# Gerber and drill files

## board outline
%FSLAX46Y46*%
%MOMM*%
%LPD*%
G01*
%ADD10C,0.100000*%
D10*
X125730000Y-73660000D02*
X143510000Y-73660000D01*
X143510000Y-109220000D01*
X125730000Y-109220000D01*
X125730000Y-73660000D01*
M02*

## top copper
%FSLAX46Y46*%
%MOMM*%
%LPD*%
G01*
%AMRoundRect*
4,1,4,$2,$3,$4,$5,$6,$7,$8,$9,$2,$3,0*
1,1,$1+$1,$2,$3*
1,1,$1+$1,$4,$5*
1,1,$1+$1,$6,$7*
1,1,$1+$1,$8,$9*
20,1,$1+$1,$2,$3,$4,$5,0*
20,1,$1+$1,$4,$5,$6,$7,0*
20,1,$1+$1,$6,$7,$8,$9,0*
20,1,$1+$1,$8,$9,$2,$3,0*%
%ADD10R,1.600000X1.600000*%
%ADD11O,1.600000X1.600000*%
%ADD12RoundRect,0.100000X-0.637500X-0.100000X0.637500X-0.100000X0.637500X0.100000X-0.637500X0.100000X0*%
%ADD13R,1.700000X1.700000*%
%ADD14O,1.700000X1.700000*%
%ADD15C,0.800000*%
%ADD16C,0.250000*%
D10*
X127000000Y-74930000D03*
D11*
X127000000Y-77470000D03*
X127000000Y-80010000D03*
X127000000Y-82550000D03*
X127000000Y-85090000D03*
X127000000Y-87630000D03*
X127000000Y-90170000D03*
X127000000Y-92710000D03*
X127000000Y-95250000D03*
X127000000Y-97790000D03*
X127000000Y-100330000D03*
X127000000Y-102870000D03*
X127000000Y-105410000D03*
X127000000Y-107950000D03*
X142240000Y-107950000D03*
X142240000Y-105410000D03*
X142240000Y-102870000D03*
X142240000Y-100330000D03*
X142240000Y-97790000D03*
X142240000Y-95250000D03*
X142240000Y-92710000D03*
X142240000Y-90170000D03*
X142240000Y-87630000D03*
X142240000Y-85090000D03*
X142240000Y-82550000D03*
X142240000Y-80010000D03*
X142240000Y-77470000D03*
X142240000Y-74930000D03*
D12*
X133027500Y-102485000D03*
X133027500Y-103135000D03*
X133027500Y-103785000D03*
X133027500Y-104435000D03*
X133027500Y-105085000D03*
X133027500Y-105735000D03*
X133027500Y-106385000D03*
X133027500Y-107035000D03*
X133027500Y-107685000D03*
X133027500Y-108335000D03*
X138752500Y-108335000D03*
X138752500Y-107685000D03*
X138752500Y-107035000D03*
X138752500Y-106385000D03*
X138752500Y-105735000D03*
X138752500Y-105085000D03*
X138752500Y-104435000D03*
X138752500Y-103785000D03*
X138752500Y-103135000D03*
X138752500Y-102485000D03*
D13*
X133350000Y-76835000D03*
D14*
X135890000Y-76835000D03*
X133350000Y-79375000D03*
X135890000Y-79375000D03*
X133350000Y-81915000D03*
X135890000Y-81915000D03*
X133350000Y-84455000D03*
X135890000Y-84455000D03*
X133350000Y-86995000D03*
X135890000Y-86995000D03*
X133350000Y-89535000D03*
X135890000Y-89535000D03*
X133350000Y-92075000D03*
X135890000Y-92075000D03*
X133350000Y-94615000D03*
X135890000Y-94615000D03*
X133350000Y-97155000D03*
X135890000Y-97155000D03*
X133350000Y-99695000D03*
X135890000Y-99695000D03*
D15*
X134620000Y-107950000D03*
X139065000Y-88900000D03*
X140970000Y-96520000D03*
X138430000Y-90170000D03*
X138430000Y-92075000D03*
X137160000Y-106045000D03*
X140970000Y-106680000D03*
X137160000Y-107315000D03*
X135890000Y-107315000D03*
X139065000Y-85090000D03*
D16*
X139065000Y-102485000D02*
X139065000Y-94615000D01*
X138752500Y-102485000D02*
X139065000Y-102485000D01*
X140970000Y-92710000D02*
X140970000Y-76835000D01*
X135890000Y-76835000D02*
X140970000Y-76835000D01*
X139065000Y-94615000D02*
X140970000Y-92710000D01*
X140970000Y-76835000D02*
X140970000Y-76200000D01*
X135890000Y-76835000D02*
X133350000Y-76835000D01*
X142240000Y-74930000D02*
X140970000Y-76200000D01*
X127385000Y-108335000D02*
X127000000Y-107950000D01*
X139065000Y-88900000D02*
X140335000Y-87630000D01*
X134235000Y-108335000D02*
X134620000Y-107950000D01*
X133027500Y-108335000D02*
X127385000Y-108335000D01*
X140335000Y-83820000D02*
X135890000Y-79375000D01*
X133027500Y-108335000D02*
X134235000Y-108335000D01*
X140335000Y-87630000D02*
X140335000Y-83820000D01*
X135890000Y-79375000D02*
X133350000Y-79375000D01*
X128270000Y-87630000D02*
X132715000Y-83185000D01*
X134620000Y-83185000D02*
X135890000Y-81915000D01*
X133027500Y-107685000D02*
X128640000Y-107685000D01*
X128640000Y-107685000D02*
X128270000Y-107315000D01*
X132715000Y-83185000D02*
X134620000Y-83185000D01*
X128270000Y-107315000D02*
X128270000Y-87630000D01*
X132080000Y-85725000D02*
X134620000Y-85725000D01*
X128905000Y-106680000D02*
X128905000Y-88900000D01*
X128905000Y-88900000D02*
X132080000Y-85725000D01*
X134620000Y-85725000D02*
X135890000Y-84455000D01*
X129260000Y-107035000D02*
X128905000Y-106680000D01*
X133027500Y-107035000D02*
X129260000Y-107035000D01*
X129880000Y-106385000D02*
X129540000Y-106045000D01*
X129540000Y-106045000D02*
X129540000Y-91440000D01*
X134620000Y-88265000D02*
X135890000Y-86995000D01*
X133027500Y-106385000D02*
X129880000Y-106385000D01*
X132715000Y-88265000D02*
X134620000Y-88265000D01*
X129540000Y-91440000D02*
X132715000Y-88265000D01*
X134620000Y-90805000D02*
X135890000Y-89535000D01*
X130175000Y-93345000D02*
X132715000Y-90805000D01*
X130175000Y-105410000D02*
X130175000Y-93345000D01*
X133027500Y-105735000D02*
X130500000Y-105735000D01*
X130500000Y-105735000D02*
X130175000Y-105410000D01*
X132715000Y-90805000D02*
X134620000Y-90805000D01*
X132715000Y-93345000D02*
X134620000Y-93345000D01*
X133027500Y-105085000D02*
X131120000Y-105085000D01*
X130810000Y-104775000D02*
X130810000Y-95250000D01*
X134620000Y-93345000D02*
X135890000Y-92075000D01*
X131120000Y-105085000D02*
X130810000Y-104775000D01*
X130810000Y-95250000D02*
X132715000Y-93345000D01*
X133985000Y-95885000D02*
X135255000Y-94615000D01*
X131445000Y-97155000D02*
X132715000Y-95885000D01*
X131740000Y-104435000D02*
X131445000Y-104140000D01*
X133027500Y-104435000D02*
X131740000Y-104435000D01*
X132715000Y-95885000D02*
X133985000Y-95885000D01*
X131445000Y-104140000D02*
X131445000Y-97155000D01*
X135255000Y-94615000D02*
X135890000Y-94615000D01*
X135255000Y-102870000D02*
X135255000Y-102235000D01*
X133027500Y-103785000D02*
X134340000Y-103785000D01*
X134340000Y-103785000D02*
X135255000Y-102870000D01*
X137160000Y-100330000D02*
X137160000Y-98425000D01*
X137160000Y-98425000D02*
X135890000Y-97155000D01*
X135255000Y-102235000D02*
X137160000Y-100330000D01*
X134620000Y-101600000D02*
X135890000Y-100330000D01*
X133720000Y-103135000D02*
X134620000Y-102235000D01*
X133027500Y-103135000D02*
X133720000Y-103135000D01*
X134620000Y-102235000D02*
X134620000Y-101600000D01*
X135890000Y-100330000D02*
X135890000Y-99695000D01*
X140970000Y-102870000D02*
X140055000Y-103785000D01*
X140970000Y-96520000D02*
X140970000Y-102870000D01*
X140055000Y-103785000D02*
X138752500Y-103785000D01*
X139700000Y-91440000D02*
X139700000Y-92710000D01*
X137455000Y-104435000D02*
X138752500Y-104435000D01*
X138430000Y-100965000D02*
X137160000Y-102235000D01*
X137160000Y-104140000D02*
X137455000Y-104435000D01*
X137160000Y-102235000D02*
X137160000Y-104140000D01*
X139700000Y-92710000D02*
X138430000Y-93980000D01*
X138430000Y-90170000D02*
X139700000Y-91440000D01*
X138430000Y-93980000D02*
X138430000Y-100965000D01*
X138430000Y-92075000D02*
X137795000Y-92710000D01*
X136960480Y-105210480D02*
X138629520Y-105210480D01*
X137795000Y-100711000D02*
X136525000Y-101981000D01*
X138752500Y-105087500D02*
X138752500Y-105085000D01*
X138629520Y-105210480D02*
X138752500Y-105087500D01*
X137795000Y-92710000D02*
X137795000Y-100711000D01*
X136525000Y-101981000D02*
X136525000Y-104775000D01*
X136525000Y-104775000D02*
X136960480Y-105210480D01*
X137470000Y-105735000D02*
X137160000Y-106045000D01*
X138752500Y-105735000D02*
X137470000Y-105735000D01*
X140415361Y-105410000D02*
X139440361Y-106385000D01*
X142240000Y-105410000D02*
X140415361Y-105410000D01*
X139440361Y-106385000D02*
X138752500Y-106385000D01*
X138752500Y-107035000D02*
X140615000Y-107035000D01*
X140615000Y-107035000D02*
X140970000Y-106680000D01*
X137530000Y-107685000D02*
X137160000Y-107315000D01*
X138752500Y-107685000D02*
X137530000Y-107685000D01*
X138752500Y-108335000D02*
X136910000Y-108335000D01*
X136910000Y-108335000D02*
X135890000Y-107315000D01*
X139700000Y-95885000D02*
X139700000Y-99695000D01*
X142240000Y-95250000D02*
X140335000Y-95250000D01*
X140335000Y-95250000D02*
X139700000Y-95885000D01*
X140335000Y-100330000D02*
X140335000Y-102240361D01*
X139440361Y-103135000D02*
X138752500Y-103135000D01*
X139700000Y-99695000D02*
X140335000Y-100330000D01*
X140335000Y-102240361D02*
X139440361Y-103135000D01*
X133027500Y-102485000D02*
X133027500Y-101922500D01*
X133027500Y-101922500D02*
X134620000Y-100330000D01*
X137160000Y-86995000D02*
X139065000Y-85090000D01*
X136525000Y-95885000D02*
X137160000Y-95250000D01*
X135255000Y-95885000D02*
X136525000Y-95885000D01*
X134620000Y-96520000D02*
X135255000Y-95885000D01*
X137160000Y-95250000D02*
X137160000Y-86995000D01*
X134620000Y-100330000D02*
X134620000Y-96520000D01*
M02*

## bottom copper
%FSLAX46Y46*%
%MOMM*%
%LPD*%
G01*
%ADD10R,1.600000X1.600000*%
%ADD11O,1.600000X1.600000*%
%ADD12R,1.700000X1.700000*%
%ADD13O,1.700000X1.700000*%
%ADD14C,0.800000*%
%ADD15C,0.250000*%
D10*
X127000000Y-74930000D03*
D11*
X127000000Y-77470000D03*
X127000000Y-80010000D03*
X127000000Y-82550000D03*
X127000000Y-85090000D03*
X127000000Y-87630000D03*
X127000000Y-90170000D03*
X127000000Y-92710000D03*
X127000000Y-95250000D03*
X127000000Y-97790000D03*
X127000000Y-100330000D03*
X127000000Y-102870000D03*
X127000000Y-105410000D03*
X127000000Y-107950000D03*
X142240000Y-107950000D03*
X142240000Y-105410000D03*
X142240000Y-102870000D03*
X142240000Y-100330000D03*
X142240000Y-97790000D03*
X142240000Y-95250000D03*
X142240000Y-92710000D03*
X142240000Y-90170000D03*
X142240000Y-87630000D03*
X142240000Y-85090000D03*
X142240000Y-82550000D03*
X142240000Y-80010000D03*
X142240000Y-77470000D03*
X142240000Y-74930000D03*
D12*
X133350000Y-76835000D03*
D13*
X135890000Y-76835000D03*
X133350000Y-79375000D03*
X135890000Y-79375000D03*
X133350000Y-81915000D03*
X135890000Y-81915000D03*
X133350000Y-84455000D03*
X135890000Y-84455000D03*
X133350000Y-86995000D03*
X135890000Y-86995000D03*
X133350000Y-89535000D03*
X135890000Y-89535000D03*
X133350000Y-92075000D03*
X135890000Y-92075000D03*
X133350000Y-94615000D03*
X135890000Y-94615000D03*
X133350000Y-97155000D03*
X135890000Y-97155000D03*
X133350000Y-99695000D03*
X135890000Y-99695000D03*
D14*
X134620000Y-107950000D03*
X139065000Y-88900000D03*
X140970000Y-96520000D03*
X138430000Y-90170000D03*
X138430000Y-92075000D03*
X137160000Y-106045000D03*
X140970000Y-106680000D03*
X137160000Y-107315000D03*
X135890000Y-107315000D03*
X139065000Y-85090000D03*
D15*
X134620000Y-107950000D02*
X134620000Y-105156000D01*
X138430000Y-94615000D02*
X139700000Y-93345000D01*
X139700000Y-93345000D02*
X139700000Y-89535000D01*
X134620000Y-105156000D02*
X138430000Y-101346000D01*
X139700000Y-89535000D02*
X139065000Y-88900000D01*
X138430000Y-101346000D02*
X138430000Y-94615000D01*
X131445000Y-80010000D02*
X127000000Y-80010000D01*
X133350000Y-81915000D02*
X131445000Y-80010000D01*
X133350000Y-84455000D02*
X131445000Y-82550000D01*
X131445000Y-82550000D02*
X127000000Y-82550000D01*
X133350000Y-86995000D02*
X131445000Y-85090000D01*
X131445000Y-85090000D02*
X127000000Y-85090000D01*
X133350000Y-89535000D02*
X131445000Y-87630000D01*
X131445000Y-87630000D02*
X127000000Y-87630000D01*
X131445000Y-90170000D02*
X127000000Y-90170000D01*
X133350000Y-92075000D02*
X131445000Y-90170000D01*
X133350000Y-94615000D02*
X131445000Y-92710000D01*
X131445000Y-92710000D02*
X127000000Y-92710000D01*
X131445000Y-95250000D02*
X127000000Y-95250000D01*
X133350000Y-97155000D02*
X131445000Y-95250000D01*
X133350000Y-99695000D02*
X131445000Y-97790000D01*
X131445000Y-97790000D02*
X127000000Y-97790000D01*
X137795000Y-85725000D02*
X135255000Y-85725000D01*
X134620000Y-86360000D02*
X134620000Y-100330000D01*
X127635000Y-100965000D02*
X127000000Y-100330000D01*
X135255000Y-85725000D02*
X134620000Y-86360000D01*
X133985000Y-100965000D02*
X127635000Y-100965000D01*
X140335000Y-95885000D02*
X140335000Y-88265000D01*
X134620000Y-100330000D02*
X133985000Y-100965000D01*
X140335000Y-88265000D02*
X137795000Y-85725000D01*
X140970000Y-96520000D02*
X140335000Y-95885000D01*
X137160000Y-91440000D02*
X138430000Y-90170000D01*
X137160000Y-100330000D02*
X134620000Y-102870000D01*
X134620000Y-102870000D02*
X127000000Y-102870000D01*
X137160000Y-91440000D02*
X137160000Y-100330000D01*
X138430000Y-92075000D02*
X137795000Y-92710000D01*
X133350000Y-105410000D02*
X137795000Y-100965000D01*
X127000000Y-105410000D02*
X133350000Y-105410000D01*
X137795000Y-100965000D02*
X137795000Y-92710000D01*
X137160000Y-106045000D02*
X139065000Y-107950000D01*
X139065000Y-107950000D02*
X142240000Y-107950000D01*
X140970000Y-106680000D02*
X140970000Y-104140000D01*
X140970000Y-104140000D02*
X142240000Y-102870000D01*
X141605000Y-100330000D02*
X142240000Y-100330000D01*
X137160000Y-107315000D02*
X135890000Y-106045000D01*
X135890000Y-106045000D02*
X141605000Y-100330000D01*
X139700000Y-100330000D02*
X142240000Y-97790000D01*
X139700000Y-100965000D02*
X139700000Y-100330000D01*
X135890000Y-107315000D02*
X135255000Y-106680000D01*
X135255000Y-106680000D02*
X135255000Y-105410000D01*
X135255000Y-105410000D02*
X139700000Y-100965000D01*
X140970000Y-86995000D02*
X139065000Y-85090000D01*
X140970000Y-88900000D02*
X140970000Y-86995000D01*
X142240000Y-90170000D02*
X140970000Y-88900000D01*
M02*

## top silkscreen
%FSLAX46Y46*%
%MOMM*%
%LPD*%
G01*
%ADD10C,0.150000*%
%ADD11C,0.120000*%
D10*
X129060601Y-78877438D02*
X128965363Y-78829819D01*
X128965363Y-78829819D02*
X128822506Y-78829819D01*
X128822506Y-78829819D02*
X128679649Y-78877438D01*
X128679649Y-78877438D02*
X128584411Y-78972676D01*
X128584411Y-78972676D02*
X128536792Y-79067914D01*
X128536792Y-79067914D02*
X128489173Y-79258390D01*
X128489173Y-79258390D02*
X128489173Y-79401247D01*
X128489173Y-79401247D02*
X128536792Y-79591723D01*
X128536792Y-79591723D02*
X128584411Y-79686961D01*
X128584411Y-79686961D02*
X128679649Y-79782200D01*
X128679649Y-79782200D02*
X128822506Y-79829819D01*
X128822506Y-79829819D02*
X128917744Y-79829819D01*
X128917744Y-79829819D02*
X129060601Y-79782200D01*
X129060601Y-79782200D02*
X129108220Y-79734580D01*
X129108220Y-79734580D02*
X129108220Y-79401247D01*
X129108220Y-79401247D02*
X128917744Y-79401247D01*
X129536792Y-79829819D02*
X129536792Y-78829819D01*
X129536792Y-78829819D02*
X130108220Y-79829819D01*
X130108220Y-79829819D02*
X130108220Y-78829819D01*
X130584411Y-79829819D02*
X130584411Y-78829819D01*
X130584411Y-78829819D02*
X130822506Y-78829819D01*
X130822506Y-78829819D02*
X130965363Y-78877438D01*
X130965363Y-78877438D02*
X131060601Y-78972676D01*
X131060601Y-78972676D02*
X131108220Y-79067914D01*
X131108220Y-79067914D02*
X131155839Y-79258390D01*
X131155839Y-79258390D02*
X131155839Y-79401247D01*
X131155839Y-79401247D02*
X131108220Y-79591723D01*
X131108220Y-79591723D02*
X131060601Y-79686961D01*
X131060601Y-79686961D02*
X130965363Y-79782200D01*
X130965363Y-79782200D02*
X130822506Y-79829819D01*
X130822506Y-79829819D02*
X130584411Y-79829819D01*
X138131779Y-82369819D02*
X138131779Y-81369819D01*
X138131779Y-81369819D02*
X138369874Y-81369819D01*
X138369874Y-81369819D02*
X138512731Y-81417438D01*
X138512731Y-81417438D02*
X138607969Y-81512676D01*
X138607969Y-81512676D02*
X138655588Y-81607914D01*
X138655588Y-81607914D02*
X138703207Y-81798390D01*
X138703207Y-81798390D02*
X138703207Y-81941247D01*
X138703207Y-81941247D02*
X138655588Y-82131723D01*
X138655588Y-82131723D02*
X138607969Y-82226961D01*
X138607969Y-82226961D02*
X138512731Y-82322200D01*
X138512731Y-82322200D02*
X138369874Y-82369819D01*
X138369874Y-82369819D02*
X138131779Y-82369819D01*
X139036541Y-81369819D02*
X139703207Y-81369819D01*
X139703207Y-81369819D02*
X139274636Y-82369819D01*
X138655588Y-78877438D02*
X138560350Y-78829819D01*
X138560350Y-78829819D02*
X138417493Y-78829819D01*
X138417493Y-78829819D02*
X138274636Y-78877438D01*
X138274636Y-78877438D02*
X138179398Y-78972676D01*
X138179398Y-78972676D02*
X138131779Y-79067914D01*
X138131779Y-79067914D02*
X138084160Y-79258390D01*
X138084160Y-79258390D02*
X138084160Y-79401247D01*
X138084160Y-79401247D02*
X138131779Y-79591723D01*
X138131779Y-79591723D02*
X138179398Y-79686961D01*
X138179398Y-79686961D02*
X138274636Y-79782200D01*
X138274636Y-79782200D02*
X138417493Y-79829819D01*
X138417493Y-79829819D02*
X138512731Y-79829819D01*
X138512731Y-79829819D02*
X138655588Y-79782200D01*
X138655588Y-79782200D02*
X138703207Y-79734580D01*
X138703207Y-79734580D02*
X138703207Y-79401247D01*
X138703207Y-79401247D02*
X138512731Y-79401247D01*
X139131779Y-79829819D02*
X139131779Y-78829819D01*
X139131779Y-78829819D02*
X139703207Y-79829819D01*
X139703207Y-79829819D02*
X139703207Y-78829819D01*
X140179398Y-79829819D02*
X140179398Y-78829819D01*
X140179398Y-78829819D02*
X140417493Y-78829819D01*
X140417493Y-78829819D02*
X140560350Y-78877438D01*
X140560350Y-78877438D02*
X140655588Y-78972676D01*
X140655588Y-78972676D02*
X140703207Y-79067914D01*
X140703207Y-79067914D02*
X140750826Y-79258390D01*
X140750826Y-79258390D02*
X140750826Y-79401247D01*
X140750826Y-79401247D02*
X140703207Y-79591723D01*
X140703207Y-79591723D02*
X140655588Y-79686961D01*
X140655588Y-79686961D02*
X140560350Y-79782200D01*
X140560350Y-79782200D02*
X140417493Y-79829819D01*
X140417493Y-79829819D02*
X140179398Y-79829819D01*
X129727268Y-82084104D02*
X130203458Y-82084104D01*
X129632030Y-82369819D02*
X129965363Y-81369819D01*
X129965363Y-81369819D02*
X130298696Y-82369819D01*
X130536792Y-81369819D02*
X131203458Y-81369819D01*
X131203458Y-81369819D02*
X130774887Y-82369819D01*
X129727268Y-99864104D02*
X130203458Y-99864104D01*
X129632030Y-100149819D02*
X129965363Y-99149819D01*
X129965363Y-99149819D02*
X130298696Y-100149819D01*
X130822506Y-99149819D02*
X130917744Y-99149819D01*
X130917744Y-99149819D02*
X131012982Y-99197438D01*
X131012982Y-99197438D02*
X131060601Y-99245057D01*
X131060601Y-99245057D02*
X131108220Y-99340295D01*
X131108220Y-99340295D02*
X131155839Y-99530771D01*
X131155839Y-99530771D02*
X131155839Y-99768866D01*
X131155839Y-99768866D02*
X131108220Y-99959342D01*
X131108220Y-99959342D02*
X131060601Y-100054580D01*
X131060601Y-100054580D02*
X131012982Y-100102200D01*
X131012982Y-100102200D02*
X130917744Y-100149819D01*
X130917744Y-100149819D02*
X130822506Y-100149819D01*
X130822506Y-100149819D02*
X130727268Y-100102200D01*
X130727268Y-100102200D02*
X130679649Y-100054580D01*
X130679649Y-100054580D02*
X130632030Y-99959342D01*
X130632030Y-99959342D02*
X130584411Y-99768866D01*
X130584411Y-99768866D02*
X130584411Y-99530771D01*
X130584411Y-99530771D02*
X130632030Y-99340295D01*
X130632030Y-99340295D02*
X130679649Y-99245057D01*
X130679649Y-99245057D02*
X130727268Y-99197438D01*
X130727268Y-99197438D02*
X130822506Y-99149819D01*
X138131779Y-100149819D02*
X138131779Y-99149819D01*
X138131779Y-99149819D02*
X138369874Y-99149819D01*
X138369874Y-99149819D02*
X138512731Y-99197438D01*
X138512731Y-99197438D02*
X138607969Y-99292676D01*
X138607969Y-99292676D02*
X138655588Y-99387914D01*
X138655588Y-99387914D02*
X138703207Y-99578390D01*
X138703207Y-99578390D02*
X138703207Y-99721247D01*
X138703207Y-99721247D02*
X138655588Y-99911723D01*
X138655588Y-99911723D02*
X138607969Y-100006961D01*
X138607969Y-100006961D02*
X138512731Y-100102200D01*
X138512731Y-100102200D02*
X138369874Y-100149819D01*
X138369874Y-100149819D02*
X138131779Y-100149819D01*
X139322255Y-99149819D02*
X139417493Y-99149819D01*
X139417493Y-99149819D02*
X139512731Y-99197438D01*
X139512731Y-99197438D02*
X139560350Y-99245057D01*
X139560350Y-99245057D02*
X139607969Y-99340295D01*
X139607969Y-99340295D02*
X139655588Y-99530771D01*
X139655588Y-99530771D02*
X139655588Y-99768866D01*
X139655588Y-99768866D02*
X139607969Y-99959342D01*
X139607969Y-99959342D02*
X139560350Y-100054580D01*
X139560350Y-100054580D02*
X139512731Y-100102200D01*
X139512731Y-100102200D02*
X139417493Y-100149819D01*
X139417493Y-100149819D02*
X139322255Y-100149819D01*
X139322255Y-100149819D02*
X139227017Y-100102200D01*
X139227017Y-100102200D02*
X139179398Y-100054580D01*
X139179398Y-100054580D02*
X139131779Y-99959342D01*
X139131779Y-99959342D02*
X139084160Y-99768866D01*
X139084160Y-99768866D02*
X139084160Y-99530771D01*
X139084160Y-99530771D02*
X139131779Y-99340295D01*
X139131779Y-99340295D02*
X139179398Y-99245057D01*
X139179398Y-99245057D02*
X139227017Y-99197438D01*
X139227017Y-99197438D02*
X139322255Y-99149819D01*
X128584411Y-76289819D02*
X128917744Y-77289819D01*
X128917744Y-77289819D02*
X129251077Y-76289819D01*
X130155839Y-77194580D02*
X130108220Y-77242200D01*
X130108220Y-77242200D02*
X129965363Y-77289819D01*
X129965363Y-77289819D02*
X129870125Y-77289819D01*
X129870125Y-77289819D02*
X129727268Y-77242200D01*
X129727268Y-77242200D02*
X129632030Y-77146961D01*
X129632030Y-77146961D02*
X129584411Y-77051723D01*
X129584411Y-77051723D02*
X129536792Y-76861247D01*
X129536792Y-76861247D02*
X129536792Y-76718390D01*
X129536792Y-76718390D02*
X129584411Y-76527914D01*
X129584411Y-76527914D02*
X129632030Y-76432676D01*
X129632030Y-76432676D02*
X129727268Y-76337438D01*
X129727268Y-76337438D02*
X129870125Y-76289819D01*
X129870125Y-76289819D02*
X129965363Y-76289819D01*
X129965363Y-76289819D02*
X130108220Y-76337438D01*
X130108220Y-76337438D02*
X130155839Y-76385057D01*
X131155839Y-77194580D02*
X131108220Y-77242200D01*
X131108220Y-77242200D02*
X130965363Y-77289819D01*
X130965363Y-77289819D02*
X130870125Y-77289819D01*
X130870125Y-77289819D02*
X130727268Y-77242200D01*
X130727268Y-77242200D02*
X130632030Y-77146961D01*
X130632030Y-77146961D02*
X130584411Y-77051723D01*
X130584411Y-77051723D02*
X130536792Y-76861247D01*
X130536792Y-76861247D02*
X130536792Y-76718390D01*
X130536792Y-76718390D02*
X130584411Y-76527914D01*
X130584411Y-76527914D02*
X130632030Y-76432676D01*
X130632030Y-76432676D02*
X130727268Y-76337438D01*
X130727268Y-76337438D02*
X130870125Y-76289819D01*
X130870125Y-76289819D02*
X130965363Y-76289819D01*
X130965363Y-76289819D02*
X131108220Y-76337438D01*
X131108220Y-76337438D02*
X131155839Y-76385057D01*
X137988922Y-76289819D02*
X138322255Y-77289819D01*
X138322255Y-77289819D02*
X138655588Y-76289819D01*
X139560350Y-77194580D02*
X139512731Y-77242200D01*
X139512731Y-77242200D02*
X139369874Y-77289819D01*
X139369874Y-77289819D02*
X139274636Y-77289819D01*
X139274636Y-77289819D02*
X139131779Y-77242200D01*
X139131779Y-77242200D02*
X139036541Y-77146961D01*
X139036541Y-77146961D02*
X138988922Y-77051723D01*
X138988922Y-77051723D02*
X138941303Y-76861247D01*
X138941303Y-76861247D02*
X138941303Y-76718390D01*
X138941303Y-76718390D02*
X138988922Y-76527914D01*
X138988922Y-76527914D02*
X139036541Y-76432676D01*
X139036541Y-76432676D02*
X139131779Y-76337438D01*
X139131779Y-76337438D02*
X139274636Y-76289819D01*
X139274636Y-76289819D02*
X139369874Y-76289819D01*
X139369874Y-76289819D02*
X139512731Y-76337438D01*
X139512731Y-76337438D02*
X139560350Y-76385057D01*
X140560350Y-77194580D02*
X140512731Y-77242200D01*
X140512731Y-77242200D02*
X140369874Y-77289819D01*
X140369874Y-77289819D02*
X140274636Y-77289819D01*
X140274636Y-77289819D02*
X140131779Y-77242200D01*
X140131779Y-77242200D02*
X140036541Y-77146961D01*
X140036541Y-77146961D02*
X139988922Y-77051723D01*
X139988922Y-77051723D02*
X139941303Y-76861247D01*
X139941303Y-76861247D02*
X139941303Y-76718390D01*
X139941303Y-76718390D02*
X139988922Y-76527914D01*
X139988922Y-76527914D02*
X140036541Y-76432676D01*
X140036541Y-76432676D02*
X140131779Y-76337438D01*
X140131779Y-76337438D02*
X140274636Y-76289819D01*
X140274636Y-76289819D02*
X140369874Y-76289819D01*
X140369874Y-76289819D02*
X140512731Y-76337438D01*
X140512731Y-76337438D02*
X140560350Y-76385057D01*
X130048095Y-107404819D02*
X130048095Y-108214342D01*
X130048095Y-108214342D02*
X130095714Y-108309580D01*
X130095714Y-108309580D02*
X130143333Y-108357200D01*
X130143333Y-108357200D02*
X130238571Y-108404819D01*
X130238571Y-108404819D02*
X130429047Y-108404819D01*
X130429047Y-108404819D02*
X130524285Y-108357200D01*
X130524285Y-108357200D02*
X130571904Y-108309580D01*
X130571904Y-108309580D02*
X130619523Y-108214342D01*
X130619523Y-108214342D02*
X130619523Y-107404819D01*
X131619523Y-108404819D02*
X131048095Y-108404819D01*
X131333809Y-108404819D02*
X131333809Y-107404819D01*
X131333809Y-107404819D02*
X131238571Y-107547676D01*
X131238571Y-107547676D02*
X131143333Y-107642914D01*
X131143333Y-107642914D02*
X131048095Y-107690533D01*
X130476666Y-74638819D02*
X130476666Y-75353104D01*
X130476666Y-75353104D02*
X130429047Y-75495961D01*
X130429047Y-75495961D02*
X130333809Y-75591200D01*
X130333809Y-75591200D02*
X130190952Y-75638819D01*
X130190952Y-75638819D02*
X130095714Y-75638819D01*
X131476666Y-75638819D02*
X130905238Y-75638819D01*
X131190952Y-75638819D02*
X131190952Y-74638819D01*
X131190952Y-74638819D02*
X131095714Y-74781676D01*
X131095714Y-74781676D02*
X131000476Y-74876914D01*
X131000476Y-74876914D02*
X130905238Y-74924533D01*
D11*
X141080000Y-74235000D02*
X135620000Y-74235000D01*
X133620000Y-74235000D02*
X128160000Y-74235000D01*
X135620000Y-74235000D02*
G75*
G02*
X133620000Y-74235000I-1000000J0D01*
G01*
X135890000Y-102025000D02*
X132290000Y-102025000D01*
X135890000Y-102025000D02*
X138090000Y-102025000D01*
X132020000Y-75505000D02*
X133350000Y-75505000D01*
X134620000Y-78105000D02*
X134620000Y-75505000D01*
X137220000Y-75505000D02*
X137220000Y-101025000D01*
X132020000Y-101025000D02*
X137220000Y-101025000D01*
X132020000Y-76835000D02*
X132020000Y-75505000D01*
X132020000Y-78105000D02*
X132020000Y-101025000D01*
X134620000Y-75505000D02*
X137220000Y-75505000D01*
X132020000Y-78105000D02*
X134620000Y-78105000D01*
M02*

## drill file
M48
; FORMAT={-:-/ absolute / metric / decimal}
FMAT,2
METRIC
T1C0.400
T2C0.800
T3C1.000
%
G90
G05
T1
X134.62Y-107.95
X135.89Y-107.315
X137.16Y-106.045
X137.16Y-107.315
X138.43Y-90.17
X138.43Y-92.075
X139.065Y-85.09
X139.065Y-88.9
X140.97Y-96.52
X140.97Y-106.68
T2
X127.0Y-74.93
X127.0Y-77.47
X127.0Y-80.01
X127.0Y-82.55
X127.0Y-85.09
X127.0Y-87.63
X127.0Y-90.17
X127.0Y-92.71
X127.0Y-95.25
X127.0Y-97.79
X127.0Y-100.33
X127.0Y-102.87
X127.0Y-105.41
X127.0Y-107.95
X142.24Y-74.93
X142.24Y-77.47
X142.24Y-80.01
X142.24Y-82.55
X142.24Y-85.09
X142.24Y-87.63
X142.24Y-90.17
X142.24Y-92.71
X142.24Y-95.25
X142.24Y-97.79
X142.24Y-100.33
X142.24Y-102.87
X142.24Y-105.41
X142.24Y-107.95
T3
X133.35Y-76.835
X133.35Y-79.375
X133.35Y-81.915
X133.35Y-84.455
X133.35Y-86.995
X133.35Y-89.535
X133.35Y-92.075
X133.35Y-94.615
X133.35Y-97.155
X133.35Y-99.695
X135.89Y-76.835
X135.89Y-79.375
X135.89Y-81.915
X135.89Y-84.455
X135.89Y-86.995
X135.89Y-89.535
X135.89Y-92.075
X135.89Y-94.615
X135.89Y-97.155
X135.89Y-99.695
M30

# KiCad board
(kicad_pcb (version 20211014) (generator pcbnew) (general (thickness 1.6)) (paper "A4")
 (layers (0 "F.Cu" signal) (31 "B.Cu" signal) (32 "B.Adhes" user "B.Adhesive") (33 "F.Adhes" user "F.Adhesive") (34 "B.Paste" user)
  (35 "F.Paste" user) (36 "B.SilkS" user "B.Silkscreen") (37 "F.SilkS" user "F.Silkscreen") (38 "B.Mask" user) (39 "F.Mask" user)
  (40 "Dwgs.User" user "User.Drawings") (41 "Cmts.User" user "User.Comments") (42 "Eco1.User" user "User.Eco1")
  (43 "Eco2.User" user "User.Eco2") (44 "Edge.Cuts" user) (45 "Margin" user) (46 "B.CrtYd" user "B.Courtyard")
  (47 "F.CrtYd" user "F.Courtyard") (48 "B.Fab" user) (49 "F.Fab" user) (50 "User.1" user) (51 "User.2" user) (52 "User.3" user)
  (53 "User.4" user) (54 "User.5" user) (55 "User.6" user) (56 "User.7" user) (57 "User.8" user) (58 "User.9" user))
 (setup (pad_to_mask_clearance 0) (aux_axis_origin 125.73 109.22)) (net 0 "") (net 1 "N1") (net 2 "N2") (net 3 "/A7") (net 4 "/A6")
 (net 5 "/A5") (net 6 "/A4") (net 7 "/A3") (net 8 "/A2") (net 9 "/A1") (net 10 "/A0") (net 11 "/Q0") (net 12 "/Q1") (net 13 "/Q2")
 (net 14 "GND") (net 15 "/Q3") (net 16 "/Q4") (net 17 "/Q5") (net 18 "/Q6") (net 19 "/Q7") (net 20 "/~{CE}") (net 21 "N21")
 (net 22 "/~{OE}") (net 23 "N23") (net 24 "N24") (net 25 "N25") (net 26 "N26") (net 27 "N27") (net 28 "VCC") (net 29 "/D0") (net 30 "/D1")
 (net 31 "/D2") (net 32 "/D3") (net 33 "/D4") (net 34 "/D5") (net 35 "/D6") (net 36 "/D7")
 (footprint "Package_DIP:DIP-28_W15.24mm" (layer "F.Cu") (at 127 74.93)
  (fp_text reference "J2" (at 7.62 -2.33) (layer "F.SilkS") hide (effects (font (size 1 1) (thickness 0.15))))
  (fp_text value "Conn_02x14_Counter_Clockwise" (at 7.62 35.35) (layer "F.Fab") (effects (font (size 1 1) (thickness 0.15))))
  (fp_line (start 14.08 -0.695) (end 8.62 -0.695) (layer "F.SilkS") (width 0.12))
  (fp_line (start 6.62 -0.695) (end 1.16 -0.695) (layer "F.SilkS") (width 0.12))
  (fp_arc (start 8.62 -0.695) (mid 7.62 0.305) (end 6.62 -0.695) (layer "F.SilkS") (width 0.12))
  (pad "1" thru_hole rect (at 0 0) (size 1.6 1.6) (drill 0.8) (layers *.Cu *.Mask) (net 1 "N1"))
  (pad "2" thru_hole oval (at 0 2.54) (size 1.6 1.6) (drill 0.8) (layers *.Cu *.Mask) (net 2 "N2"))
  (pad "3" thru_hole oval (at 0 5.08) (size 1.6 1.6) (drill 0.8) (layers *.Cu *.Mask) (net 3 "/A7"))
  (pad "4" thru_hole oval (at 0 7.62) (size 1.6 1.6) (drill 0.8) (layers *.Cu *.Mask) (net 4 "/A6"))
  (pad "5" thru_hole oval (at 0 10.16) (size 1.6 1.6) (drill 0.8) (layers *.Cu *.Mask) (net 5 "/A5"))
  (pad "6" thru_hole oval (at 0 12.7) (size 1.6 1.6) (drill 0.8) (layers *.Cu *.Mask) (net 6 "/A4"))
  (pad "7" thru_hole oval (at 0 15.24) (size 1.6 1.6) (drill 0.8) (layers *.Cu *.Mask) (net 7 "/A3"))
  (pad "8" thru_hole oval (at 0 17.78) (size 1.6 1.6) (drill 0.8) (layers *.Cu *.Mask) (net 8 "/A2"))
  (pad "9" thru_hole oval (at 0 20.32) (size 1.6 1.6) (drill 0.8) (layers *.Cu *.Mask) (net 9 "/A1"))
  (pad "10" thru_hole oval (at 0 22.86) (size 1.6 1.6) (drill 0.8) (layers *.Cu *.Mask) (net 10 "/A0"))
  (pad "11" thru_hole oval (at 0 25.4) (size 1.6 1.6) (drill 0.8) (layers *.Cu *.Mask) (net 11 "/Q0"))
  (pad "12" thru_hole oval (at 0 27.94) (size 1.6 1.6) (drill 0.8) (layers *.Cu *.Mask) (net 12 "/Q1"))
  (pad "13" thru_hole oval (at 0 30.48) (size 1.6 1.6) (drill 0.8) (layers *.Cu *.Mask) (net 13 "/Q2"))
  (pad "14" thru_hole oval (at 0 33.02) (size 1.6 1.6) (drill 0.8) (layers *.Cu *.Mask) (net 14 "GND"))
  (pad "15" thru_hole oval (at 15.24 33.02) (size 1.6 1.6) (drill 0.8) (layers *.Cu *.Mask) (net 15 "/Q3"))
  (pad "16" thru_hole oval (at 15.24 30.48) (size 1.6 1.6) (drill 0.8) (layers *.Cu *.Mask) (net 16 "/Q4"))
  (pad "17" thru_hole oval (at 15.24 27.94) (size 1.6 1.6) (drill 0.8) (layers *.Cu *.Mask) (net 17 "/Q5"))
  (pad "18" thru_hole oval (at 15.24 25.4) (size 1.6 1.6) (drill 0.8) (layers *.Cu *.Mask) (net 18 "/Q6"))
  (pad "19" thru_hole oval (at 15.24 22.86) (size 1.6 1.6) (drill 0.8) (layers *.Cu *.Mask) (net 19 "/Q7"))
  (pad "20" thru_hole oval (at 15.24 20.32) (size 1.6 1.6) (drill 0.8) (layers *.Cu *.Mask) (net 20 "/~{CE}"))
  (pad "21" thru_hole oval (at 15.24 17.78) (size 1.6 1.6) (drill 0.8) (layers *.Cu *.Mask) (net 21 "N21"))
  (pad "22" thru_hole oval (at 15.24 15.24) (size 1.6 1.6) (drill 0.8) (layers *.Cu *.Mask) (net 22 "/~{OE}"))
  (pad "23" thru_hole oval (at 15.24 12.7) (size 1.6 1.6) (drill 0.8) (layers *.Cu *.Mask) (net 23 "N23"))
  (pad "24" thru_hole oval (at 15.24 10.16) (size 1.6 1.6) (drill 0.8) (layers *.Cu *.Mask) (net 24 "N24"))
  (pad "25" thru_hole oval (at 15.24 7.62) (size 1.6 1.6) (drill 0.8) (layers *.Cu *.Mask) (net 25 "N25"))
  (pad "26" thru_hole oval (at 15.24 5.08) (size 1.6 1.6) (drill 0.8) (layers *.Cu *.Mask) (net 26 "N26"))
  (pad "27" thru_hole oval (at 15.24 2.54) (size 1.6 1.6) (drill 0.8) (layers *.Cu *.Mask) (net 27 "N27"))
  (pad "28" thru_hole oval (at 15.24 0) (size 1.6 1.6) (drill 0.8) (layers *.Cu *.Mask) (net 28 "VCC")))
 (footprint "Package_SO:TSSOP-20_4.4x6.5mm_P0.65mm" (layer "F.Cu") (at 135.89 105.41)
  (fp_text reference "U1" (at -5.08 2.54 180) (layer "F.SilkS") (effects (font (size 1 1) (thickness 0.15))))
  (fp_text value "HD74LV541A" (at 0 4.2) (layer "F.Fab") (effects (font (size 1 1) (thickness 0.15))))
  (fp_line (start 0 -3.385) (end -3.6 -3.385) (layer "F.SilkS") (width 0.12))
  (fp_line (start 0 -3.385) (end 2.2 -3.385) (layer "F.SilkS") (width 0.12))
  (pad "1" smd roundrect (at -2.8625 -2.925) (size 1.475 0.4) (layers "F.Cu" "F.Paste" "F.Mask") (roundrect_rratio 0.25) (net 22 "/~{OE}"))
  (pad "2" smd roundrect (at -2.8625 -2.275) (size 1.475 0.4) (layers "F.Cu" "F.Paste" "F.Mask") (roundrect_rratio 0.25) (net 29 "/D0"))
  (pad "3" smd roundrect (at -2.8625 -1.625) (size 1.475 0.4) (layers "F.Cu" "F.Paste" "F.Mask") (roundrect_rratio 0.25) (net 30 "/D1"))
  (pad "4" smd roundrect (at -2.8625 -0.975) (size 1.475 0.4) (layers "F.Cu" "F.Paste" "F.Mask") (roundrect_rratio 0.25) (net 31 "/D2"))
  (pad "5" smd roundrect (at -2.8625 -0.325) (size 1.475 0.4) (layers "F.Cu" "F.Paste" "F.Mask") (roundrect_rratio 0.25) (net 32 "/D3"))
  (pad "6" smd roundrect (at -2.8625 0.325) (size 1.475 0.4) (layers "F.Cu" "F.Paste" "F.Mask") (roundrect_rratio 0.25) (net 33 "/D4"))
  (pad "7" smd roundrect (at -2.8625 0.975) (size 1.475 0.4) (layers "F.Cu" "F.Paste" "F.Mask") (roundrect_rratio 0.25) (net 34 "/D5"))
  (pad "8" smd roundrect (at -2.8625 1.625) (size 1.475 0.4) (layers "F.Cu" "F.Paste" "F.Mask") (roundrect_rratio 0.25) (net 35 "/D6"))
  (pad "9" smd roundrect (at -2.8625 2.275) (size 1.475 0.4) (layers "F.Cu" "F.Paste" "F.Mask") (roundrect_rratio 0.25) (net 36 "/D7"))
  (pad "10" smd roundrect (at -2.8625 2.925) (size 1.475 0.4) (layers "F.Cu" "F.Paste" "F.Mask") (roundrect_rratio 0.25) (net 14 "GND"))
  (pad "11" smd roundrect (at 2.8625 2.925) (size 1.475 0.4) (layers "F.Cu" "F.Paste" "F.Mask") (roundrect_rratio 0.25) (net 19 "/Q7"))
  (pad "12" smd roundrect (at 2.8625 2.275) (size 1.475 0.4) (layers "F.Cu" "F.Paste" "F.Mask") (roundrect_rratio 0.25) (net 18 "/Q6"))
  (pad "13" smd roundrect (at 2.8625 1.625) (size 1.475 0.4) (layers "F.Cu" "F.Paste" "F.Mask") (roundrect_rratio 0.25) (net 17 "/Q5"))
  (pad "14" smd roundrect (at 2.8625 0.975) (size 1.475 0.4) (layers "F.Cu" "F.Paste" "F.Mask") (roundrect_rratio 0.25) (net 16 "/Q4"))
  (pad "15" smd roundrect (at 2.8625 0.325) (size 1.475 0.4) (layers "F.Cu" "F.Paste" "F.Mask") (roundrect_rratio 0.25) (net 15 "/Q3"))
  (pad "16" smd roundrect (at 2.8625 -0.325) (size 1.475 0.4) (layers "F.Cu" "F.Paste" "F.Mask") (roundrect_rratio 0.25) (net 13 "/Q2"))
  (pad "17" smd roundrect (at 2.8625 -0.975) (size 1.475 0.4) (layers "F.Cu" "F.Paste" "F.Mask") (roundrect_rratio 0.25) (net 12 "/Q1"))
  (pad "18" smd roundrect (at 2.8625 -1.625) (size 1.475 0.4) (layers "F.Cu" "F.Paste" "F.Mask") (roundrect_rratio 0.25) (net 11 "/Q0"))
  (pad "19" smd roundrect (at 2.8625 -2.275) (size 1.475 0.4) (layers "F.Cu" "F.Paste" "F.Mask") (roundrect_rratio 0.25) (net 20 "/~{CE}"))
  (pad "20" smd roundrect (at 2.8625 -2.925) (size 1.475 0.4) (layers "F.Cu" "F.Paste" "F.Mask") (roundrect_rratio 0.25) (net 28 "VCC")))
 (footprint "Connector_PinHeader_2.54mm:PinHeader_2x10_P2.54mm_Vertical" (layer "F.Cu") (at 133.35 76.835)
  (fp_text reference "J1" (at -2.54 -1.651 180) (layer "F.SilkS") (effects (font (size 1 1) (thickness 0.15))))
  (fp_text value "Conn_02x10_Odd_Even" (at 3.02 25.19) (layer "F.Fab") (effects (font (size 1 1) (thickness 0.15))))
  (fp_line (start -1.33 -1.33) (end 0 -1.33) (layer "F.SilkS") (width 0.12))
  (fp_line (start 1.27 1.27) (end 1.27 -1.33) (layer "F.SilkS") (width 0.12))
  (fp_line (start 3.87 -1.33) (end 3.87 24.19) (layer "F.SilkS") (width 0.12))
  (fp_line (start -1.33 24.19) (end 3.87 24.19) (layer "F.SilkS") (width 0.12))
  (fp_line (start -1.33 0) (end -1.33 -1.33) (layer "F.SilkS") (width 0.12))
  (fp_line (start -1.33 1.27) (end -1.33 24.19) (layer "F.SilkS") (width 0.12))
  (fp_line (start 1.27 -1.33) (end 3.87 -1.33) (layer "F.SilkS") (width 0.12))
  (fp_line (start -1.33 1.27) (end 1.27 1.27) (layer "F.SilkS") (width 0.12))
  (pad "1" thru_hole rect (at 0 0) (size 1.7 1.7) (drill 1) (layers *.Cu *.Mask) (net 28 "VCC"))
  (pad "2" thru_hole oval (at 2.54 0) (size 1.7 1.7) (drill 1) (layers *.Cu *.Mask) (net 28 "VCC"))
  (pad "3" thru_hole oval (at 0 2.54) (size 1.7 1.7) (drill 1) (layers *.Cu *.Mask) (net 14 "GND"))
  (pad "4" thru_hole oval (at 2.54 2.54) (size 1.7 1.7) (drill 1) (layers *.Cu *.Mask) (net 14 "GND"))
  (pad "5" thru_hole oval (at 0 5.08) (size 1.7 1.7) (drill 1) (layers *.Cu *.Mask) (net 3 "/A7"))
  (pad "6" thru_hole oval (at 2.54 5.08) (size 1.7 1.7) (drill 1) (layers *.Cu *.Mask) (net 36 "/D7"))
  (pad "7" thru_hole oval (at 0 7.62) (size 1.7 1.7) (drill 1) (layers *.Cu *.Mask) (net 4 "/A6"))
  (pad "8" thru_hole oval (at 2.54 7.62) (size 1.7 1.7) (drill 1) (layers *.Cu *.Mask) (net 35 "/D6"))
  (pad "9" thru_hole oval (at 0 10.16) (size 1.7 1.7) (drill 1) (layers *.Cu *.Mask) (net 5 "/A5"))
  (pad "10" thru_hole oval (at 2.54 10.16) (size 1.7 1.7) (drill 1) (layers *.Cu *.Mask) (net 34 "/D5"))
  (pad "11" thru_hole oval (at 0 12.7) (size 1.7 1.7) (drill 1) (layers *.Cu *.Mask) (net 6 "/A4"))
  (pad "12" thru_hole oval (at 2.54 12.7) (size 1.7 1.7) (drill 1) (layers *.Cu *.Mask) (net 33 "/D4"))
  (pad "13" thru_hole oval (at 0 15.24) (size 1.7 1.7) (drill 1) (layers *.Cu *.Mask) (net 7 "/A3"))
  (pad "14" thru_hole oval (at 2.54 15.24) (size 1.7 1.7) (drill 1) (layers *.Cu *.Mask) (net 32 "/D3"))
  (pad "15" thru_hole oval (at 0 17.78) (size 1.7 1.7) (drill 1) (layers *.Cu *.Mask) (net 8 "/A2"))
  (pad "16" thru_hole oval (at 2.54 17.78) (size 1.7 1.7) (drill 1) (layers *.Cu *.Mask) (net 31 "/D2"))
  (pad "17" thru_hole oval (at 0 20.32) (size 1.7 1.7) (drill 1) (layers *.Cu *.Mask) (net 9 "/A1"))
  (pad "18" thru_hole oval (at 2.54 20.32) (size 1.7 1.7) (drill 1) (layers *.Cu *.Mask) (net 30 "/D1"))
  (pad "19" thru_hole oval (at 0 22.86) (size 1.7 1.7) (drill 1) (layers *.Cu *.Mask) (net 10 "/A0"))
  (pad "20" thru_hole oval (at 2.54 22.86) (size 1.7 1.7) (drill 1) (layers *.Cu *.Mask) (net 29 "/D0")))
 (gr_rect (start 125.73 73.66) (end 143.51 109.22) (layer "Edge.Cuts") (width 0.1) (fill none))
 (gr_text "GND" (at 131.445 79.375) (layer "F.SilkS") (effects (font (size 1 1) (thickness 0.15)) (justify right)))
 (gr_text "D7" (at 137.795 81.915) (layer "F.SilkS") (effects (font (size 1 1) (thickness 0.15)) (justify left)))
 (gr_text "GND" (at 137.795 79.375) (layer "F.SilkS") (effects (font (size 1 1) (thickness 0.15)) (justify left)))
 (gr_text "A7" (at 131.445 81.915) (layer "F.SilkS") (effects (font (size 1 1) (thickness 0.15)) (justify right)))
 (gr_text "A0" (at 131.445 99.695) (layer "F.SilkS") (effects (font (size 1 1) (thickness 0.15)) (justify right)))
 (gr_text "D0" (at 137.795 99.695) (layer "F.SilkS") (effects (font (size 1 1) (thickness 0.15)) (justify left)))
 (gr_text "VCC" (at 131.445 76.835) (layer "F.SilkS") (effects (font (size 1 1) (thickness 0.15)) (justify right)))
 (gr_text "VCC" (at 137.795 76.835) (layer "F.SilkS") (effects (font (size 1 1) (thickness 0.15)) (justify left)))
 (segment (start 139.065 102.485) (end 139.065 94.615) (width 0.25) (layer "F.Cu") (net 28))
 (segment (start 138.7525 102.485) (end 139.065 102.485) (width 0.25) (layer "F.Cu") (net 28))
 (segment (start 140.97 92.71) (end 140.97 76.835) (width 0.25) (layer "F.Cu") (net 28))
 (segment (start 135.89 76.835) (end 140.97 76.835) (width 0.25) (layer "F.Cu") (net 28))
 (segment (start 139.065 94.615) (end 140.97 92.71) (width 0.25) (layer "F.Cu") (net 28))
 (segment (start 140.97 76.835) (end 140.97 76.2) (width 0.25) (layer "F.Cu") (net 28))
 (segment (start 135.89 76.835) (end 133.35 76.835) (width 0.25) (layer "F.Cu") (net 28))
 (segment (start 142.24 74.93) (end 140.97 76.2) (width 0.25) (layer "F.Cu") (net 28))
 (segment (start 127.385 108.335) (end 127 107.95) (width 0.25) (layer "F.Cu") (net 14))
 (segment (start 139.065 88.9) (end 140.335 87.63) (width 0.25) (layer "F.Cu") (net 14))
 (segment (start 134.235 108.335) (end 134.62 107.95) (width 0.25) (layer "F.Cu") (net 14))
 (segment (start 133.0275 108.335) (end 127.385 108.335) (width 0.25) (layer "F.Cu") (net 14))
 (segment (start 140.335 83.82) (end 135.89 79.375) (width 0.25) (layer "F.Cu") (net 14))
 (segment (start 133.0275 108.335) (end 134.235 108.335) (width 0.25) (layer "F.Cu") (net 14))
 (segment (start 140.335 87.63) (end 140.335 83.82) (width 0.25) (layer "F.Cu") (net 14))
 (segment (start 135.89 79.375) (end 133.35 79.375) (width 0.25) (layer "F.Cu") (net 14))
 (via (at 134.62 107.95) (size 0.8) (drill 0.4) (layers "F.Cu" "B.Cu") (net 14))
 (via (at 139.065 88.9) (size 0.8) (drill 0.4) (layers "F.Cu" "B.Cu") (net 14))
 (segment (start 134.62 107.95) (end 134.62 105.156) (width 0.25) (layer "B.Cu") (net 14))
 (segment (start 138.43 94.615) (end 139.7 93.345) (width 0.25) (layer "B.Cu") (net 14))
 (segment (start 139.7 93.345) (end 139.7 89.535) (width 0.25) (layer "B.Cu") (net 14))
 (segment (start 134.62 105.156) (end 138.43 101.346) (width 0.25) (layer "B.Cu") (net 14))
 (segment (start 139.7 89.535) (end 139.065 88.9) (width 0.25) (layer "B.Cu") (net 14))
 (segment (start 138.43 101.346) (end 138.43 94.615) (width 0.25) (layer "B.Cu") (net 14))
 (segment (start 131.445 80.01) (end 127 80.01) (width 0.25) (layer "B.Cu") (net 3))
 (segment (start 133.35 81.915) (end 131.445 80.01) (width 0.25) (layer "B.Cu") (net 3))
 (segment (start 128.27 87.63) (end 132.715 83.185) (width 0.25) (layer "F.Cu") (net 36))
 (segment (start 134.62 83.185) (end 135.89 81.915) (width 0.25) (layer "F.Cu") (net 36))
 (segment (start 133.0275 107.685) (end 128.64 107.685) (width 0.25) (layer "F.Cu") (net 36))
 (segment (start 128.64 107.685) (end 128.27 107.315) (width 0.25) (layer "F.Cu") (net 36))
 (segment (start 132.715 83.185) (end 134.62 83.185) (width 0.25) (layer "F.Cu") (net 36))
 (segment (start 128.27 107.315) (end 128.27 87.63) (width 0.25) (layer "F.Cu") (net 36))
 (segment (start 133.35 84.455) (end 131.445 82.55) (width 0.25) (layer "B.Cu") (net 4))
 (segment (start 131.445 82.55) (end 127 82.55) (width 0.25) (layer "B.Cu") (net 4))
 (segment (start 132.08 85.725) (end 134.62 85.725) (width 0.25) (layer "F.Cu") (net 35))
 (segment (start 128.905 106.68) (end 128.905 88.9) (width 0.25) (layer "F.Cu") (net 35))
 (segment (start 128.905 88.9) (end 132.08 85.725) (width 0.25) (layer "F.Cu") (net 35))
 (segment (start 134.62 85.725) (end 135.89 84.455) (width 0.25) (layer "F.Cu") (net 35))
 (segment (start 129.26 107.035) (end 128.905 106.68) (width 0.25) (layer "F.Cu") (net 35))
 (segment (start 133.0275 107.035) (end 129.26 107.035) (width 0.25) (layer "F.Cu") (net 35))
 (segment (start 133.35 86.995) (end 131.445 85.09) (width 0.25) (layer "B.Cu") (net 5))
 (segment (start 131.445 85.09) (end 127 85.09) (width 0.25) (layer "B.Cu") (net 5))
 (segment (start 129.88 106.385) (end 129.54 106.045) (width 0.25) (layer "F.Cu") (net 34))
 (segment (start 129.54 106.045) (end 129.54 91.44) (width 0.25) (layer "F.Cu") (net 34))
 (segment (start 134.62 88.265) (end 135.89 86.995) (width 0.25) (layer "F.Cu") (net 34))
 (segment (start 133.0275 106.385) (end 129.88 106.385) (width 0.25) (layer "F.Cu") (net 34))
 (segment (start 132.715 88.265) (end 134.62 88.265) (width 0.25) (layer "F.Cu") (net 34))
 (segment (start 129.54 91.44) (end 132.715 88.265) (width 0.25) (layer "F.Cu") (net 34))
 (segment (start 133.35 89.535) (end 131.445 87.63) (width 0.25) (layer "B.Cu") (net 6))
 (segment (start 131.445 87.63) (end 127 87.63) (width 0.25) (layer "B.Cu") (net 6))
 (segment (start 134.62 90.805) (end 135.89 89.535) (width 0.25) (layer "F.Cu") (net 33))
 (segment (start 130.175 93.345) (end 132.715 90.805) (width 0.25) (layer "F.Cu") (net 33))
 (segment (start 130.175 105.41) (end 130.175 93.345) (width 0.25) (layer "F.Cu") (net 33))
 (segment (start 133.0275 105.735) (end 130.5 105.735) (width 0.25) (layer "F.Cu") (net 33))
 (segment (start 130.5 105.735) (end 130.175 105.41) (width 0.25) (layer "F.Cu") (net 33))
 (segment (start 132.715 90.805) (end 134.62 90.805) (width 0.25) (layer "F.Cu") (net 33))
 (segment (start 131.445 90.17) (end 127 90.17) (width 0.25) (layer "B.Cu") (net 7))
 (segment (start 133.35 92.075) (end 131.445 90.17) (width 0.25) (layer "B.Cu") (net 7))
 (segment (start 132.715 93.345) (end 134.62 93.345) (width 0.25) (layer "F.Cu") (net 32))
 (segment (start 133.0275 105.085) (end 131.12 105.085) (width 0.25) (layer "F.Cu") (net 32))
 (segment (start 130.81 104.775) (end 130.81 95.25) (width 0.25) (layer "F.Cu") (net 32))
 (segment (start 134.62 93.345) (end 135.89 92.075) (width 0.25) (layer "F.Cu") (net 32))
 (segment (start 131.12 105.085) (end 130.81 104.775) (width 0.25) (layer "F.Cu") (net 32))
 (segment (start 130.81 95.25) (end 132.715 93.345) (width 0.25) (layer "F.Cu") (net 32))
 (segment (start 133.35 94.615) (end 131.445 92.71) (width 0.25) (layer "B.Cu") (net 8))
 (segment (start 131.445 92.71) (end 127 92.71) (width 0.25) (layer "B.Cu") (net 8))
 (segment (start 133.985 95.885) (end 135.255 94.615) (width 0.25) (layer "F.Cu") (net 31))
 (segment (start 131.445 97.155) (end 132.715 95.885) (width 0.25) (layer "F.Cu") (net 31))
 (segment (start 131.74 104.435) (end 131.445 104.14) (width 0.25) (layer "F.Cu") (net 31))
 (segment (start 133.0275 104.435) (end 131.74 104.435) (width 0.25) (layer "F.Cu") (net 31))
 (segment (start 132.715 95.885) (end 133.985 95.885) (width 0.25) (layer "F.Cu") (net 31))
 (segment (start 131.445 104.14) (end 131.445 97.155) (width 0.25) (layer "F.Cu") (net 31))
 (segment (start 135.255 94.615) (end 135.89 94.615) (width 0.25) (layer "F.Cu") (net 31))
 (segment (start 131.445 95.25) (end 127 95.25) (width 0.25) (layer "B.Cu") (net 9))
 (segment (start 133.35 97.155) (end 131.445 95.25) (width 0.25) (layer "B.Cu") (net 9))
 (segment (start 135.255 102.87) (end 135.255 102.235) (width 0.25) (layer "F.Cu") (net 30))
 (segment (start 133.0275 103.785) (end 134.34 103.785) (width 0.25) (layer "F.Cu") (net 30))
 (segment (start 134.34 103.785) (end 135.255 102.87) (width 0.25) (layer "F.Cu") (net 30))
 (segment (start 137.16 100.33) (end 137.16 98.425) (width 0.25) (layer "F.Cu") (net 30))
 (segment (start 137.16 98.425) (end 135.89 97.155) (width 0.25) (layer "F.Cu") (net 30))
 (segment (start 135.255 102.235) (end 137.16 100.33) (width 0.25) (layer "F.Cu") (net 30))
 (segment (start 133.35 99.695) (end 131.445 97.79) (width 0.25) (layer "B.Cu") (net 10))
 (segment (start 131.445 97.79) (end 127 97.79) (width 0.25) (layer "B.Cu") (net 10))
 (segment (start 134.62 101.6) (end 135.89 100.33) (width 0.25) (layer "F.Cu") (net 29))
 (segment (start 133.72 103.135) (end 134.62 102.235) (width 0.25) (layer "F.Cu") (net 29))
 (segment (start 133.0275 103.135) (end 133.72 103.135) (width 0.25) (layer "F.Cu") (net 29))
 (segment (start 134.62 102.235) (end 134.62 101.6) (width 0.25) (layer "F.Cu") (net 29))
 (segment (start 135.89 100.33) (end 135.89 99.695) (width 0.25) (layer "F.Cu") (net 29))
 (segment (start 140.97 102.87) (end 140.055 103.785) (width 0.25) (layer "F.Cu") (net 11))
 (segment (start 140.97 96.52) (end 140.97 102.87) (width 0.25) (layer "F.Cu") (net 11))
 (segment (start 140.055 103.785) (end 138.7525 103.785) (width 0.25) (layer "F.Cu") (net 11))
 (via (at 140.97 96.52) (size 0.8) (drill 0.4) (layers "F.Cu" "B.Cu") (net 11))
 (segment (start 137.795 85.725) (end 135.255 85.725) (width 0.25) (layer "B.Cu") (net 11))
 (segment (start 134.62 86.36) (end 134.62 100.33) (width 0.25) (layer "B.Cu") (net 11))
 (segment (start 127.635 100.965) (end 127 100.33) (width 0.25) (layer "B.Cu") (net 11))
 (segment (start 135.255 85.725) (end 134.62 86.36) (width 0.25) (layer "B.Cu") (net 11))
 (segment (start 133.985 100.965) (end 127.635 100.965) (width 0.25) (layer "B.Cu") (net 11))
 (segment (start 140.335 95.885) (end 140.335 88.265) (width 0.25) (layer "B.Cu") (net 11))
 (segment (start 134.62 100.33) (end 133.985 100.965) (width 0.25) (layer "B.Cu") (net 11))
 (segment (start 140.335 88.265) (end 137.795 85.725) (width 0.25) (layer "B.Cu") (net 11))
 (segment (start 140.97 96.52) (end 140.335 95.885) (width 0.25) (layer "B.Cu") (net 11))
 (segment (start 139.7 91.44) (end 139.7 92.71) (width 0.25) (layer "F.Cu") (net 12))
 (segment (start 137.455 104.435) (end 138.7525 104.435) (width 0.25) (layer "F.Cu") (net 12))
 (segment (start 138.43 100.965) (end 137.16 102.235) (width 0.25) (layer "F.Cu") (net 12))
 (segment (start 137.16 104.14) (end 137.455 104.435) (width 0.25) (layer "F.Cu") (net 12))
 (segment (start 137.16 102.235) (end 137.16 104.14) (width 0.25) (layer "F.Cu") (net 12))
 (segment (start 139.7 92.71) (end 138.43 93.98) (width 0.25) (layer "F.Cu") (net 12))
 (segment (start 138.43 90.17) (end 139.7 91.44) (width 0.25) (layer "F.Cu") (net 12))
 (segment (start 138.43 93.98) (end 138.43 100.965) (width 0.25) (layer "F.Cu") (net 12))
 (via (at 138.43 90.17) (size 0.8) (drill 0.4) (layers "F.Cu" "B.Cu") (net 12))
 (segment (start 137.16 91.44) (end 138.43 90.17) (width 0.25) (layer "B.Cu") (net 12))
 (segment (start 137.16 100.33) (end 134.62 102.87) (width 0.25) (layer "B.Cu") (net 12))
 (segment (start 134.62 102.87) (end 127 102.87) (width 0.25) (layer "B.Cu") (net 12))
 (segment (start 137.16 91.44) (end 137.16 100.33) (width 0.25) (layer "B.Cu") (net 12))
 (segment (start 138.43 92.075) (end 137.795 92.71) (width 0.25) (layer "F.Cu") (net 13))
 (segment (start 136.96048 105.21048) (end 138.62952 105.21048) (width 0.25) (layer "F.Cu") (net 13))
 (segment (start 137.795 100.711) (end 136.525 101.981) (width 0.25) (layer "F.Cu") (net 13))
 (segment (start 138.7525 105.0875) (end 138.7525 105.085) (width 0.25) (layer "F.Cu") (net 13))
 (segment (start 138.62952 105.21048) (end 138.7525 105.0875) (width 0.25) (layer "F.Cu") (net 13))
 (segment (start 137.795 92.71) (end 137.795 100.711) (width 0.25) (layer "F.Cu") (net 13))
 (segment (start 136.525 101.981) (end 136.525 104.775) (width 0.25) (layer "F.Cu") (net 13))
 (segment (start 136.525 104.775) (end 136.96048 105.21048) (width 0.25) (layer "F.Cu") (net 13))
 (via (at 138.43 92.075) (size 0.8) (drill 0.4) (layers "F.Cu" "B.Cu") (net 13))
 (segment (start 138.43 92.075) (end 137.795 92.71) (width 0.25) (layer "B.Cu") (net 13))
 (segment (start 133.35 105.41) (end 137.795 100.965) (width 0.25) (layer "B.Cu") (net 13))
 (segment (start 127 105.41) (end 133.35 105.41) (width 0.25) (layer "B.Cu") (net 13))
 (segment (start 137.795 100.965) (end 137.795 92.71) (width 0.25) (layer "B.Cu") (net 13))
 (segment (start 137.47 105.735) (end 137.16 106.045) (width 0.25) (layer "F.Cu") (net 15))
 (segment (start 138.7525 105.735) (end 137.47 105.735) (width 0.25) (layer "F.Cu") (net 15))
 (via (at 137.16 106.045) (size 0.8) (drill 0.4) (layers "F.Cu" "B.Cu") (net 15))
 (segment (start 137.16 106.045) (end 139.065 107.95) (width 0.25) (layer "B.Cu") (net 15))
 (segment (start 139.065 107.95) (end 142.24 107.95) (width 0.25) (layer "B.Cu") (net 15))
 (segment (start 140.415361 105.41) (end 139.440361 106.385) (width 0.25) (layer "F.Cu") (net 16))
 (segment (start 142.24 105.41) (end 140.415361 105.41) (width 0.25) (layer "F.Cu") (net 16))
 (segment (start 139.440361 106.385) (end 138.7525 106.385) (width 0.25) (layer "F.Cu") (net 16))
 (segment (start 138.7525 107.035) (end 140.615 107.035) (width 0.25) (layer "F.Cu") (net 17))
 (segment (start 140.615 107.035) (end 140.97 106.68) (width 0.25) (layer "F.Cu") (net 17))
 (via (at 140.97 106.68) (size 0.8) (drill 0.4) (layers "F.Cu" "B.Cu") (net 17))
 (segment (start 140.97 106.68) (end 140.97 104.14) (width 0.25) (layer "B.Cu") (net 17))
 (segment (start 140.97 104.14) (end 142.24 102.87) (width 0.25) (layer "B.Cu") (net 17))
 (segment (start 137.53 107.685) (end 137.16 107.315) (width 0.25) (layer "F.Cu") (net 18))
 (segment (start 138.7525 107.685) (end 137.53 107.685) (width 0.25) (layer "F.Cu") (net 18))
 (via (at 137.16 107.315) (size 0.8) (drill 0.4) (layers "F.Cu" "B.Cu") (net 18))
 (segment (start 141.605 100.33) (end 142.24 100.33) (width 0.25) (layer "B.Cu") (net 18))
 (segment (start 137.16 107.315) (end 135.89 106.045) (width 0.25) (layer "B.Cu") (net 18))
 (segment (start 135.89 106.045) (end 141.605 100.33) (width 0.25) (layer "B.Cu") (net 18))
 (segment (start 138.7525 108.335) (end 136.91 108.335) (width 0.25) (layer "F.Cu") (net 19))
 (segment (start 136.91 108.335) (end 135.89 107.315) (width 0.25) (layer "F.Cu") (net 19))
 (via (at 135.89 107.315) (size 0.8) (drill 0.4) (layers "F.Cu" "B.Cu") (free) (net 19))
 (segment (start 139.7 100.33) (end 142.24 97.79) (width 0.25) (layer "B.Cu") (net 19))
 (segment (start 139.7 100.965) (end 139.7 100.33) (width 0.25) (layer "B.Cu") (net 19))
 (segment (start 135.89 107.315) (end 135.255 106.68) (width 0.25) (layer "B.Cu") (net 19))
 (segment (start 135.255 106.68) (end 135.255 105.41) (width 0.25) (layer "B.Cu") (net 19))
 (segment (start 135.255 105.41) (end 139.7 100.965) (width 0.25) (layer "B.Cu") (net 19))
 (segment (start 139.7 95.885) (end 139.7 99.695) (width 0.25) (layer "F.Cu") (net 20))
 (segment (start 142.24 95.25) (end 140.335 95.25) (width 0.25) (layer "F.Cu") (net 20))
 (segment (start 140.335 95.25) (end 139.7 95.885) (width 0.25) (layer "F.Cu") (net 20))
 (segment (start 140.335 100.33) (end 140.335 102.240361) (width 0.25) (layer "F.Cu") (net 20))
 (segment (start 139.440361 103.135) (end 138.7525 103.135) (width 0.25) (layer "F.Cu") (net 20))
 (segment (start 139.7 99.695) (end 140.335 100.33) (width 0.25) (layer "F.Cu") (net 20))
 (segment (start 140.335 102.240361) (end 139.440361 103.135) (width 0.25) (layer "F.Cu") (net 20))
 (segment (start 133.0275 102.485) (end 133.0275 101.9225) (width 0.25) (layer "F.Cu") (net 22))
 (segment (start 133.0275 101.9225) (end 134.62 100.33) (width 0.25) (layer "F.Cu") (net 22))
 (segment (start 137.16 86.995) (end 139.065 85.09) (width 0.25) (layer "F.Cu") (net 22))
 (segment (start 136.525 95.885) (end 137.16 95.25) (width 0.25) (layer "F.Cu") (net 22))
 (segment (start 135.255 95.885) (end 136.525 95.885) (width 0.25) (layer "F.Cu") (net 22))
 (segment (start 134.62 96.52) (end 135.255 95.885) (width 0.25) (layer "F.Cu") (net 22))
 (segment (start 137.16 95.25) (end 137.16 86.995) (width 0.25) (layer "F.Cu") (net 22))
 (segment (start 134.62 100.33) (end 134.62 96.52) (width 0.25) (layer "F.Cu") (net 22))
 (via (at 139.065 85.09) (size 0.8) (drill 0.4) (layers "F.Cu" "B.Cu") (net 22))
 (segment (start 140.97 86.995) (end 139.065 85.09) (width 0.25) (layer "B.Cu") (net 22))
 (segment (start 140.97 88.9) (end 140.97 86.995) (width 0.25) (layer "B.Cu") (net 22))
 (segment (start 142.24 90.17) (end 140.97 88.9) (width 0.25) (layer "B.Cu") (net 22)))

